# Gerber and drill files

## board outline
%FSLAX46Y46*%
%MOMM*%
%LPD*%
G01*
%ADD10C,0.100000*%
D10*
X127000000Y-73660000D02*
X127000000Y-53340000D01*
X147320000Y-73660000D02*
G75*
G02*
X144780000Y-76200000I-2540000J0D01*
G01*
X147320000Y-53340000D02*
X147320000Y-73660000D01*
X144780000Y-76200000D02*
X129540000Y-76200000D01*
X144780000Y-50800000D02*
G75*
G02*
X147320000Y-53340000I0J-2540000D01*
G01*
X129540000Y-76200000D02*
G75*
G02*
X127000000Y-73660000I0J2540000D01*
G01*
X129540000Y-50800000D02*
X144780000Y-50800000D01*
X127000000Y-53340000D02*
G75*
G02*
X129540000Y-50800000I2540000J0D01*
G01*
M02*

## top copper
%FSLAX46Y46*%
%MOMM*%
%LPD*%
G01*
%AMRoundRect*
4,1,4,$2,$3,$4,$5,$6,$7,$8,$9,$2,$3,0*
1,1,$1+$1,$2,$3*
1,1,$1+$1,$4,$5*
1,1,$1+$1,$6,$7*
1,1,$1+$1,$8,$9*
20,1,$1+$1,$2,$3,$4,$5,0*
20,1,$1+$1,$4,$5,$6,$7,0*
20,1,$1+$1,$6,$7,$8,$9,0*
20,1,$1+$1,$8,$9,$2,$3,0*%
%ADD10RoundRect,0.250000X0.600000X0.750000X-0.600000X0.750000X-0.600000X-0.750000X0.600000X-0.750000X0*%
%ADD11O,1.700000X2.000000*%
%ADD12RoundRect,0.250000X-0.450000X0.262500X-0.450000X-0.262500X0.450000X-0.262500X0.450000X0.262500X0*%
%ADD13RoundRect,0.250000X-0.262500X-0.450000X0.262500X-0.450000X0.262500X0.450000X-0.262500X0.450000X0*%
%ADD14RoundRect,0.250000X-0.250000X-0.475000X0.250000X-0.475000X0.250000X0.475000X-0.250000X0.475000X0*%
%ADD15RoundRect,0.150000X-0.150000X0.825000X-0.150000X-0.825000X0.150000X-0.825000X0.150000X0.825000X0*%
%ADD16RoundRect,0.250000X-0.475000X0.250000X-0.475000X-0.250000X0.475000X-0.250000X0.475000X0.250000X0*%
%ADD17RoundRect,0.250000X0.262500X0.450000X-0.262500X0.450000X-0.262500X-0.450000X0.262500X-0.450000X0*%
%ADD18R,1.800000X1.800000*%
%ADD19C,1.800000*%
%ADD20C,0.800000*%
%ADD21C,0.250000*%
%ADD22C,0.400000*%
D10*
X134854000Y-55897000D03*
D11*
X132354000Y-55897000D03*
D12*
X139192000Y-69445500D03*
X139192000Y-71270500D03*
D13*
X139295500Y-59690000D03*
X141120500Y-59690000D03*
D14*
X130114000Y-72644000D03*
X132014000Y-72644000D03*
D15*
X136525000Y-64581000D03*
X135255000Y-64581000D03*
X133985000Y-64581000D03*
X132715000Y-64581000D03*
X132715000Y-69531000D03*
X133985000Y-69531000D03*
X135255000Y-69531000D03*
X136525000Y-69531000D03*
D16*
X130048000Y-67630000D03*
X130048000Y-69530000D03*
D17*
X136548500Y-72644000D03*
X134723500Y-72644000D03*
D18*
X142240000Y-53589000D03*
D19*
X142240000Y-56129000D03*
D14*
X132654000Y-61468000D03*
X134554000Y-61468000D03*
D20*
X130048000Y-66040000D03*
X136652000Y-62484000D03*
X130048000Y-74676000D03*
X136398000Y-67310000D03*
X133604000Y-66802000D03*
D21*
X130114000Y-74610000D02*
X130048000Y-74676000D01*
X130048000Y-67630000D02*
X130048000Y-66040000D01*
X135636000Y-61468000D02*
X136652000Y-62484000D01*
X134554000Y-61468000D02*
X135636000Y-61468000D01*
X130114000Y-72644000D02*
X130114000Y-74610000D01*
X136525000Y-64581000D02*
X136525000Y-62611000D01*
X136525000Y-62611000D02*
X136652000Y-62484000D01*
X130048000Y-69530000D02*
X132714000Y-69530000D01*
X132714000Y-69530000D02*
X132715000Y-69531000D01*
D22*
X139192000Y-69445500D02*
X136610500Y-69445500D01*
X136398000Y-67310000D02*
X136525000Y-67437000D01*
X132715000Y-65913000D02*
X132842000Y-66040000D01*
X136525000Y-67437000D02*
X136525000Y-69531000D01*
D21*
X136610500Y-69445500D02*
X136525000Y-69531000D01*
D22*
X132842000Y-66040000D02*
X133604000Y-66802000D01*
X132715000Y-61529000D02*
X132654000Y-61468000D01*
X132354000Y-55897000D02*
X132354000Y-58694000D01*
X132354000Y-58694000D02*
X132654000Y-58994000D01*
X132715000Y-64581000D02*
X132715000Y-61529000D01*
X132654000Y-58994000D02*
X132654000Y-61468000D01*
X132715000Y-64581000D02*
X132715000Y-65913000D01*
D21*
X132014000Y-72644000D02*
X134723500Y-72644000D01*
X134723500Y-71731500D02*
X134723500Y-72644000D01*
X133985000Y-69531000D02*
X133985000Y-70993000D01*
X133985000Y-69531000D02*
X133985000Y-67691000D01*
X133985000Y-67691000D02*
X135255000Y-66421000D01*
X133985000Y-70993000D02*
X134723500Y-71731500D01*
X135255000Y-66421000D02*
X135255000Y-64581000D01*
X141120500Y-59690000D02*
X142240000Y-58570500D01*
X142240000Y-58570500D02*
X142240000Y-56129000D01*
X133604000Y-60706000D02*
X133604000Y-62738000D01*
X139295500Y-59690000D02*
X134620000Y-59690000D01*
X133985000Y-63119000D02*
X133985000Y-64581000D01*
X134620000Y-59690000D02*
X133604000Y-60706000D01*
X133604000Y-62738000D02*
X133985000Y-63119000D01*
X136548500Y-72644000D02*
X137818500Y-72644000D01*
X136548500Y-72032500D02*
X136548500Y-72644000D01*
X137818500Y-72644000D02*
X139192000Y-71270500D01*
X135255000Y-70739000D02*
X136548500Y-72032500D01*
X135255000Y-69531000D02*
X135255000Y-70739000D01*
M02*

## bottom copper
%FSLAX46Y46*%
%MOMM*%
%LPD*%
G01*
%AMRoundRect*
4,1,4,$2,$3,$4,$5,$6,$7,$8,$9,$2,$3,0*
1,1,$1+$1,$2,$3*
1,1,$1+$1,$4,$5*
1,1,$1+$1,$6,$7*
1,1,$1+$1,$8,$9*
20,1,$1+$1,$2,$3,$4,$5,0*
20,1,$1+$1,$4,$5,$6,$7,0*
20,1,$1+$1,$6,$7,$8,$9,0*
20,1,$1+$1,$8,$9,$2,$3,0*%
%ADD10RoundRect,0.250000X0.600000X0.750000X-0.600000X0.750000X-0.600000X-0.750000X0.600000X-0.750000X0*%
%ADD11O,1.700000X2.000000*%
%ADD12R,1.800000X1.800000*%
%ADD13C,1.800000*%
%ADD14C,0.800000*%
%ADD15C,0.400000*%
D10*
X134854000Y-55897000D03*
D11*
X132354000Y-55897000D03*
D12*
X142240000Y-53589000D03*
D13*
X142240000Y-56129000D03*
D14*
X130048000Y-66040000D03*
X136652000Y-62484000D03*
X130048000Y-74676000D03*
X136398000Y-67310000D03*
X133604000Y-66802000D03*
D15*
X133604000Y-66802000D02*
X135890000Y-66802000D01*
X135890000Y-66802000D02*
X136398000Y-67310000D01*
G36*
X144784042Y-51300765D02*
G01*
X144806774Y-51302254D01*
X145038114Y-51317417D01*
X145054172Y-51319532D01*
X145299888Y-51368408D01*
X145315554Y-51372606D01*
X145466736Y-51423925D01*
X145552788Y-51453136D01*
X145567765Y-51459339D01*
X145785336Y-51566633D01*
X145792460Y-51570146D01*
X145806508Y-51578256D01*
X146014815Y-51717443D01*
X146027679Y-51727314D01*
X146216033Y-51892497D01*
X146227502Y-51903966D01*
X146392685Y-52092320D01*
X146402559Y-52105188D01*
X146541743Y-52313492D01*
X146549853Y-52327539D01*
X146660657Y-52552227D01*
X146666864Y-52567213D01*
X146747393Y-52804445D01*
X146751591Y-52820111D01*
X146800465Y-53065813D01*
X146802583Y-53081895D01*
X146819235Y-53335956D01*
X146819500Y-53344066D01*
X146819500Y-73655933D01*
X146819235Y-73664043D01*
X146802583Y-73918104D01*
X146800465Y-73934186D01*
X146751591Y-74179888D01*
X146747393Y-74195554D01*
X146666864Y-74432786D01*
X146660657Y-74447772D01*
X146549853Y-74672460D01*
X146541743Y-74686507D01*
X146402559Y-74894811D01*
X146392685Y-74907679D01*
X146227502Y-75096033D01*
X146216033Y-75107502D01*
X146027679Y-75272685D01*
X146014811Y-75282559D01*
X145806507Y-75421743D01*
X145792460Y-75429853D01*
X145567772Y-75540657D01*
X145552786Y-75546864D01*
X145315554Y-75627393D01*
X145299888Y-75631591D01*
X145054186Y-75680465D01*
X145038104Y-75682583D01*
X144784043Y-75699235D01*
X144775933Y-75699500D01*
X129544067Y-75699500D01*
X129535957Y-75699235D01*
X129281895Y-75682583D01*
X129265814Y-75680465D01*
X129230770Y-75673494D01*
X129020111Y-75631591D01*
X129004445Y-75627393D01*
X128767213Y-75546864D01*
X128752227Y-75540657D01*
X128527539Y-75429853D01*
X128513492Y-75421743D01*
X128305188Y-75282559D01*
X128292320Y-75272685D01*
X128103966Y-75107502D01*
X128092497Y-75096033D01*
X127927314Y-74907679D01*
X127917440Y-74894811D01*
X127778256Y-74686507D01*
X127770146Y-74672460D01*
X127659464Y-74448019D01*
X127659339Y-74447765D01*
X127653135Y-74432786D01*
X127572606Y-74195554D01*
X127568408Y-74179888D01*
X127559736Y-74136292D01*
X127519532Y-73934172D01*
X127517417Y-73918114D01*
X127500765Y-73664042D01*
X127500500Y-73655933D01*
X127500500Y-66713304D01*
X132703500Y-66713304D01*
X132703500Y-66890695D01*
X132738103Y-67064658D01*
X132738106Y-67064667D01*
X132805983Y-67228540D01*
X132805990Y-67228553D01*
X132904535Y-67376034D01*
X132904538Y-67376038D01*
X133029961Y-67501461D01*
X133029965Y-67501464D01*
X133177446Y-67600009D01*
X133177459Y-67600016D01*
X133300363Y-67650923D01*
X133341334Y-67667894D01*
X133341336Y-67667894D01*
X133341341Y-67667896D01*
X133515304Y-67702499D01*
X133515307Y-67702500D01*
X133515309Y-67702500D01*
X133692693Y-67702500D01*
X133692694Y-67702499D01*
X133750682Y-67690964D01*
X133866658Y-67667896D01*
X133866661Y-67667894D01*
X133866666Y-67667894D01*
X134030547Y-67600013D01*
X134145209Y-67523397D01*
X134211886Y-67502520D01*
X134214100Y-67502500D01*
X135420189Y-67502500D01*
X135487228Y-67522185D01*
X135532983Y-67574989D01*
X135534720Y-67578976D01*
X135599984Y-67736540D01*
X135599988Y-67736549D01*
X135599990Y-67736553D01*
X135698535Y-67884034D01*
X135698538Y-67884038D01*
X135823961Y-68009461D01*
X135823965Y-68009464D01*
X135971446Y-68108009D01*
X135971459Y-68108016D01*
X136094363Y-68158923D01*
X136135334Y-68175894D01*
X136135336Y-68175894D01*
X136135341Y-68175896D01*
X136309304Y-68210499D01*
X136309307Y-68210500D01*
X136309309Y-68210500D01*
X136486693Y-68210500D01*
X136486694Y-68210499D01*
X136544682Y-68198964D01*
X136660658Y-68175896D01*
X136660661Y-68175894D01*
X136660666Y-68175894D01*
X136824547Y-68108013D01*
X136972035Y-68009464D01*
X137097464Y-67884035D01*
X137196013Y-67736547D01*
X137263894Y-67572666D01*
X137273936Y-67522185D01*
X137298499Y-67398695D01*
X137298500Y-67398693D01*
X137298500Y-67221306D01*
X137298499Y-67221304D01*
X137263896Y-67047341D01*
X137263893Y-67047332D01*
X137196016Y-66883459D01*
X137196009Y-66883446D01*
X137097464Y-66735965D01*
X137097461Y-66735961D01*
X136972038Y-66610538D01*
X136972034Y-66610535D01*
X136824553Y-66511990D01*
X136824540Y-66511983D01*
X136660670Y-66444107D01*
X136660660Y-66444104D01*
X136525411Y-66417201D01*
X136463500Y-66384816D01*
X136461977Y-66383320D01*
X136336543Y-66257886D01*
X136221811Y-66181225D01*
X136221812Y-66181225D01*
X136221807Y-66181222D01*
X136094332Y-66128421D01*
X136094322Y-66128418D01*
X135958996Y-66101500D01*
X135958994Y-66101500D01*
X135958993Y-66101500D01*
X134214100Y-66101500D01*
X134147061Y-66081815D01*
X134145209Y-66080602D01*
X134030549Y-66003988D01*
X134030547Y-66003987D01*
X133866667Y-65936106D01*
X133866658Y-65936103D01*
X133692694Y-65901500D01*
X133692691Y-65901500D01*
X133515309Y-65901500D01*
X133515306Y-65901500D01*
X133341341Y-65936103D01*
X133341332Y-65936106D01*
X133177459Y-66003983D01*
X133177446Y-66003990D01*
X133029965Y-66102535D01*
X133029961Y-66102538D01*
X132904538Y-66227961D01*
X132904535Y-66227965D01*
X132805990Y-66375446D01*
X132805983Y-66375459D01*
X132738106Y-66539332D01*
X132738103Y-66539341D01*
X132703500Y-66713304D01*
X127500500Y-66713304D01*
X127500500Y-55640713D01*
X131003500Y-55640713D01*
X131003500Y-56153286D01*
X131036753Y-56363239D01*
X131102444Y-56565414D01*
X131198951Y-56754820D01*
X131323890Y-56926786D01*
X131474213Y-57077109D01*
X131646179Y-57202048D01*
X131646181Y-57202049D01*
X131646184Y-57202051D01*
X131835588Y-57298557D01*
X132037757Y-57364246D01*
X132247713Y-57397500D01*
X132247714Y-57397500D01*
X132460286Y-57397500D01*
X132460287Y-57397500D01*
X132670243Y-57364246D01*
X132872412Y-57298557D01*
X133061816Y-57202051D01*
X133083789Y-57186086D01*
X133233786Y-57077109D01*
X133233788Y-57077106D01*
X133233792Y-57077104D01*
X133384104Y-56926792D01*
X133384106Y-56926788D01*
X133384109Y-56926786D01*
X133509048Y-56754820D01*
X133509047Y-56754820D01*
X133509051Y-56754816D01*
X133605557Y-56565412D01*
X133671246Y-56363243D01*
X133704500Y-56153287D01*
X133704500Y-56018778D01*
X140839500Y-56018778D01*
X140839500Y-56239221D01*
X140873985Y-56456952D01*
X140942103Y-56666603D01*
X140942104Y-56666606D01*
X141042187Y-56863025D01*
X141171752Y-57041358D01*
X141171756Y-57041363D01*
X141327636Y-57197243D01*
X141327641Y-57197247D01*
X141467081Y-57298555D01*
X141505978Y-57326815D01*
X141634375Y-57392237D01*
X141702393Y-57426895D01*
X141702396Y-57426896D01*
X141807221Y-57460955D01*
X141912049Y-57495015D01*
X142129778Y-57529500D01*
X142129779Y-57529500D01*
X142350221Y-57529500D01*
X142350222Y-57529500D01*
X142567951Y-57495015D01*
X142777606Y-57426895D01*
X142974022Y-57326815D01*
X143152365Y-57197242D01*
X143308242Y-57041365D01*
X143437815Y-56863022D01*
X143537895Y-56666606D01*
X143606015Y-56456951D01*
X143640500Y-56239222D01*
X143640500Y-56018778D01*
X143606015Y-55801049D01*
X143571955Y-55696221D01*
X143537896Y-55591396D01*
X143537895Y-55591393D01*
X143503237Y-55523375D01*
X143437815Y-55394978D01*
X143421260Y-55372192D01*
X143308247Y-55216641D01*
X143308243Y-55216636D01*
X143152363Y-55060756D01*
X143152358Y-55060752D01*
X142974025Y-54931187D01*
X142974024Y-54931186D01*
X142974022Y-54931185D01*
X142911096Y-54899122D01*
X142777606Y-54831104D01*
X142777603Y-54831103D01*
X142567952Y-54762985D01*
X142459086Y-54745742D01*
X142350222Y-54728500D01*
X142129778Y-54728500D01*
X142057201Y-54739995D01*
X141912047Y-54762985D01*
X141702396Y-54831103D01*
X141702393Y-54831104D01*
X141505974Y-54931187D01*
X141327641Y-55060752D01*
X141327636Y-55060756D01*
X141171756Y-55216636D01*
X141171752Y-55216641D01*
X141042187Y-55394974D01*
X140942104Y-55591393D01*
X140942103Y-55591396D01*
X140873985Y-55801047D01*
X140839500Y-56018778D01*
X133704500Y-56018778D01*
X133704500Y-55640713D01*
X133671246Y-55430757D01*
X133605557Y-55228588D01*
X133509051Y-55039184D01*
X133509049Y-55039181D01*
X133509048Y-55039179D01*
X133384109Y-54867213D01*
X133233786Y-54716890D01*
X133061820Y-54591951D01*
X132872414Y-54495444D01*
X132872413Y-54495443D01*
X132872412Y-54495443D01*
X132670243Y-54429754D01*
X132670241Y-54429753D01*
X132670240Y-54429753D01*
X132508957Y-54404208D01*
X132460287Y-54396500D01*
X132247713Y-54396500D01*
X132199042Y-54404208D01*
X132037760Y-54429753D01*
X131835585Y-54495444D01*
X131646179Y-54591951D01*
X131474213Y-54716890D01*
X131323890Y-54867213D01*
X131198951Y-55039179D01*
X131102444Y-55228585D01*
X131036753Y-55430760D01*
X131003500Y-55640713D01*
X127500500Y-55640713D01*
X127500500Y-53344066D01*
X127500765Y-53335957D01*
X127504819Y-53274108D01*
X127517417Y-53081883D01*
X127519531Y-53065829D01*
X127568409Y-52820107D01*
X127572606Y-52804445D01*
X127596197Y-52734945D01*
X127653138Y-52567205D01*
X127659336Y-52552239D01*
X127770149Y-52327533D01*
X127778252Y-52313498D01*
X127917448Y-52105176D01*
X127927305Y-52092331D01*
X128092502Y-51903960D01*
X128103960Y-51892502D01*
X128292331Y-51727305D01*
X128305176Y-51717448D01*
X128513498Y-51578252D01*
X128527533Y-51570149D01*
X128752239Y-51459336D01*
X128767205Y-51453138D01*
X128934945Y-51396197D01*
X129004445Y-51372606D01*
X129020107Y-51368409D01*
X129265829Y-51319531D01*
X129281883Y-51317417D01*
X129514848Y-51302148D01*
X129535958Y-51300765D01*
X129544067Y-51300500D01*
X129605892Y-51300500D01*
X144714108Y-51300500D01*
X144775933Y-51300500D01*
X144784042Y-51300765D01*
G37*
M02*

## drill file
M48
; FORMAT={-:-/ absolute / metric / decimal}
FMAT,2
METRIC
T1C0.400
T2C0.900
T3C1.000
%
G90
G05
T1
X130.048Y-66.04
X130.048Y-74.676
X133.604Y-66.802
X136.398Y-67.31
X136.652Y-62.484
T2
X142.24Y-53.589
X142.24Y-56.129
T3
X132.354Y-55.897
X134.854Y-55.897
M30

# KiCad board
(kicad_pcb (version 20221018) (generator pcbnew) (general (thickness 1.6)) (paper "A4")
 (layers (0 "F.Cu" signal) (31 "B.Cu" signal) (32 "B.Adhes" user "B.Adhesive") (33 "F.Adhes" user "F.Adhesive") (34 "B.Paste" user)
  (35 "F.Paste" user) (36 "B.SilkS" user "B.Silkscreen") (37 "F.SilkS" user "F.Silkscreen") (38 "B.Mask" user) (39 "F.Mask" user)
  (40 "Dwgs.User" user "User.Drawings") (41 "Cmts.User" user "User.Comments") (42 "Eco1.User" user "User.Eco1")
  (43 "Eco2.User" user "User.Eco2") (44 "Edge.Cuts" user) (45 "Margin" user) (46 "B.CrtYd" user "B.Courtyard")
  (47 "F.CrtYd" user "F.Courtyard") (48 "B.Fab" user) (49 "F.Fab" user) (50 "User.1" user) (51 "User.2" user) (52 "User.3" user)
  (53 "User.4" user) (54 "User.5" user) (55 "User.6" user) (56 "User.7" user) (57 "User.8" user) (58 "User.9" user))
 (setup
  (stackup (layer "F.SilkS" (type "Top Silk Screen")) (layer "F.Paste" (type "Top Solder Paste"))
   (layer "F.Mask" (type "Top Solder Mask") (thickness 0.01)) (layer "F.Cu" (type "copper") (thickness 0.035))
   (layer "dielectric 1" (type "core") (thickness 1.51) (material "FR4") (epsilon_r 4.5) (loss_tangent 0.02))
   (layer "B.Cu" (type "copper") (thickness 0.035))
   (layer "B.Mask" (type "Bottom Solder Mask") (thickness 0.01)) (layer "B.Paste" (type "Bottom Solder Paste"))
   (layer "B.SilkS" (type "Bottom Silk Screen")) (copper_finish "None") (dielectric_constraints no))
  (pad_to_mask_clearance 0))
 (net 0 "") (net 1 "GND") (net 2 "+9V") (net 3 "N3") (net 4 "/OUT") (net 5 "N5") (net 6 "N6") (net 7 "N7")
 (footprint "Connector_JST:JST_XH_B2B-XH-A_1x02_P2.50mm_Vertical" (layer "F.Cu") (at 134.854 55.897 180)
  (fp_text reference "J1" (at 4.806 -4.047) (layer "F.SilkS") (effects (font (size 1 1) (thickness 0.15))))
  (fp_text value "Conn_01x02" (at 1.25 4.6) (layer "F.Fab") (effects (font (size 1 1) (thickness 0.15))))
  (pad "1" thru_hole roundrect (at 0 0 180) (size 1.7 2) (drill 1) (layers "*.Cu" "*.Mask") (roundrect_rratio 0.1470588235) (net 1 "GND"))
  (pad "2" thru_hole oval (at 2.5 0 180) (size 1.7 2) (drill 1) (layers "*.Cu" "*.Mask") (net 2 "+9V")))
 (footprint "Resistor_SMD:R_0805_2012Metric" (layer "F.Cu") (at 139.192 70.358 -90)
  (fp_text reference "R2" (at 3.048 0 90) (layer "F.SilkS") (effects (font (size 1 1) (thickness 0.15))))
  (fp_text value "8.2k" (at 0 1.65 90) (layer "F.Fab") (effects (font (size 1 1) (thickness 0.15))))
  (pad "1" smd roundrect (at -0.9125 0 270) (size 1.025 1.4) (layers "F.Cu" "F.Paste" "F.Mask") (roundrect_rratio 0.243902439) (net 2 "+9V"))
  (pad "2" smd roundrect (at 0.9125 0 270) (size 1.025 1.4) (layers "F.Cu" "F.Paste" "F.Mask") (roundrect_rratio 0.243902439) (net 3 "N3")))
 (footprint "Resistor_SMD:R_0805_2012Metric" (layer "F.Cu") (at 140.208 59.69)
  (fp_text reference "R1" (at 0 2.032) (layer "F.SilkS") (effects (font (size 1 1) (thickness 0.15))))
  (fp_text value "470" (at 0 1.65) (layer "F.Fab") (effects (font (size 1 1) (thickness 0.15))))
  (pad "1" smd roundrect (at -0.9125 0) (size 1.025 1.4) (layers "F.Cu" "F.Paste" "F.Mask") (roundrect_rratio 0.243902439) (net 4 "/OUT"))
  (pad "2" smd roundrect (at 0.9125 0) (size 1.025 1.4) (layers "F.Cu" "F.Paste" "F.Mask") (roundrect_rratio 0.243902439) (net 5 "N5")))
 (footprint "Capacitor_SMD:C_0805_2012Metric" (layer "F.Cu") (at 131.064 72.644)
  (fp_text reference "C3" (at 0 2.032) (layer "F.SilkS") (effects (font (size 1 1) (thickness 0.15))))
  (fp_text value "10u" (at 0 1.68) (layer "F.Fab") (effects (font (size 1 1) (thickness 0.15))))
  (pad "1" smd roundrect (at -0.95 0) (size 1 1.45) (layers "F.Cu" "F.Paste" "F.Mask") (roundrect_rratio 0.25) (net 1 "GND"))
  (pad "2" smd roundrect (at 0.95 0) (size 1 1.45) (layers "F.Cu" "F.Paste" "F.Mask") (roundrect_rratio 0.25) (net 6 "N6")))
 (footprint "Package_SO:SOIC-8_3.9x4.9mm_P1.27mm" (layer "F.Cu") (at 134.62 67.056 -90)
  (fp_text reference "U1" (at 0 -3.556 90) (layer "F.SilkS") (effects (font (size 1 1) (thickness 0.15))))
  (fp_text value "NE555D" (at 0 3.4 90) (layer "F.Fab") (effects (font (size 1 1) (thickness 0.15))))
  (pad "1" smd roundrect (at -2.475 -1.905 270) (size 1.95 0.6) (layers "F.Cu" "F.Paste" "F.Mask") (roundrect_rratio 0.25) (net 1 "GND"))
  (pad "2" smd roundrect (at -2.475 -0.635 270) (size 1.95 0.6) (layers "F.Cu" "F.Paste" "F.Mask") (roundrect_rratio 0.25) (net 6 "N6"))
  (pad "3" smd roundrect (at -2.475 0.635 270) (size 1.95 0.6) (layers "F.Cu" "F.Paste" "F.Mask") (roundrect_rratio 0.25) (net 4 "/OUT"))
  (pad "4" smd roundrect (at -2.475 1.905 270) (size 1.95 0.6) (layers "F.Cu" "F.Paste" "F.Mask") (roundrect_rratio 0.25) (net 2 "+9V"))
  (pad "5" smd roundrect (at 2.475 1.905 270) (size 1.95 0.6) (layers "F.Cu" "F.Paste" "F.Mask") (roundrect_rratio 0.25) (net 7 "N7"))
  (pad "6" smd roundrect (at 2.475 0.635 270) (size 1.95 0.6) (layers "F.Cu" "F.Paste" "F.Mask") (roundrect_rratio 0.25) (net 6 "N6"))
  (pad "7" smd roundrect (at 2.475 -0.635 270) (size 1.95 0.6) (layers "F.Cu" "F.Paste" "F.Mask") (roundrect_rratio 0.25) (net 3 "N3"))
  (pad "8" smd roundrect (at 2.475 -1.905 270) (size 1.95 0.6) (layers "F.Cu" "F.Paste" "F.Mask") (roundrect_rratio 0.25) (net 2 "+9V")))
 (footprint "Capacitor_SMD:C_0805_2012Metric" (layer "F.Cu") (at 130.048 68.58 -90)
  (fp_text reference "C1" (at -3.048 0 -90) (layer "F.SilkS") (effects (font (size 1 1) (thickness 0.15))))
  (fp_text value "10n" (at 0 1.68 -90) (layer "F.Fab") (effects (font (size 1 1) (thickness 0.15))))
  (pad "1" smd roundrect (at -0.95 0 270) (size 1 1.45) (layers "F.Cu" "F.Paste" "F.Mask") (roundrect_rratio 0.25) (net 1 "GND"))
  (pad "2" smd roundrect (at 0.95 0 270) (size 1 1.45) (layers "F.Cu" "F.Paste" "F.Mask") (roundrect_rratio 0.25) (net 7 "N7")))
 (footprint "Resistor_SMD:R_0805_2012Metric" (layer "F.Cu") (at 135.636 72.644 180)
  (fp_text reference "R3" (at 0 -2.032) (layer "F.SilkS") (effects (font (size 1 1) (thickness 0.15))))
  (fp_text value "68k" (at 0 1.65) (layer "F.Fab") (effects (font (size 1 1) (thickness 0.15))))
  (pad "1" smd roundrect (at -0.9125 0 180) (size 1.025 1.4) (layers "F.Cu" "F.Paste" "F.Mask") (roundrect_rratio 0.243902439) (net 3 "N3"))
  (pad "2" smd roundrect (at 0.9125 0 180) (size 1.025 1.4) (layers "F.Cu" "F.Paste" "F.Mask") (roundrect_rratio 0.243902439) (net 6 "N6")))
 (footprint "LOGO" (layer "F.Cu") (at 142.748 67.31 90)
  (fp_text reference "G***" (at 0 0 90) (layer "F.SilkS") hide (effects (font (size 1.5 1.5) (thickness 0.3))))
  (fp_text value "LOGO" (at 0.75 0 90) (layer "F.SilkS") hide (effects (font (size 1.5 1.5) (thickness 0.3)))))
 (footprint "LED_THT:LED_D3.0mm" (layer "F.Cu") (at 142.24 53.589 -90)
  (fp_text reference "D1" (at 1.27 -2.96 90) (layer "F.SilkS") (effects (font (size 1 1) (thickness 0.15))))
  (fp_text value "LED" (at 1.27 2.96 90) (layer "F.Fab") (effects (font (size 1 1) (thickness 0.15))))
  (pad "1" thru_hole rect (at 0 0 270) (size 1.8 1.8) (drill 0.9) (layers "*.Cu" "*.Mask") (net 1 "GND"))
  (pad "2" thru_hole circle (at 2.54 0 270) (size 1.8 1.8) (drill 0.9) (layers "*.Cu" "*.Mask") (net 5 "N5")))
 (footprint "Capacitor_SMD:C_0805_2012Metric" (layer "F.Cu") (at 133.604 61.468)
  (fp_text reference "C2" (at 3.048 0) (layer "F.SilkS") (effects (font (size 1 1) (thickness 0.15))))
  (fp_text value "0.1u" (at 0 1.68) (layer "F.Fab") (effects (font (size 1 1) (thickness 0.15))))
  (pad "1" smd roundrect (at -0.95 0) (size 1 1.45) (layers "F.Cu" "F.Paste" "F.Mask") (roundrect_rratio 0.25) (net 2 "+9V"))
  (pad "2" smd roundrect (at 0.95 0) (size 1 1.45) (layers "F.Cu" "F.Paste" "F.Mask") (roundrect_rratio 0.25) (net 1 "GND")))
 (gr_line (start 127 73.66) (end 127 53.34) (stroke (width 0.1) (type default)) (layer "Edge.Cuts"))
 (gr_arc (start 147.32 73.66) (mid 146.576051 75.456051) (end 144.78 76.2) (stroke (width 0.1) (type default)) (layer "Edge.Cuts"))
 (gr_line (start 147.32 53.34) (end 147.32 73.66) (stroke (width 0.1) (type default)) (layer "Edge.Cuts"))
 (gr_line (start 144.78 76.2) (end 129.54 76.2) (stroke (width 0.1) (type default)) (layer "Edge.Cuts"))
 (gr_arc (start 144.78 50.8) (mid 146.576051 51.543949) (end 147.32 53.34) (stroke (width 0.1) (type default)) (layer "Edge.Cuts"))
 (gr_arc (start 129.54 76.2) (mid 127.743949 75.456051) (end 127 73.66) (stroke (width 0.1) (type default)) (layer "Edge.Cuts"))
 (gr_line (start 129.54 50.8) (end 144.78 50.8) (stroke (width 0.1) (type default)) (layer "Edge.Cuts"))
 (gr_arc (start 127 53.34) (mid 127.743949 51.543949) (end 129.54 50.8) (stroke (width 0.1) (type default)) (layer "Edge.Cuts"))
 (segment (start 130.114 74.61) (end 130.048 74.676) (width 0.25) (layer "F.Cu") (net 1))
 (segment (start 130.048 67.63) (end 130.048 66.04) (width 0.25) (layer "F.Cu") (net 1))
 (segment (start 135.636 61.468) (end 136.652 62.484) (width 0.25) (layer "F.Cu") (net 1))
 (segment (start 134.554 61.468) (end 135.636 61.468) (width 0.25) (layer "F.Cu") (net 1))
 (segment (start 130.114 72.644) (end 130.114 74.61) (width 0.25) (layer "F.Cu") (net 1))
 (segment (start 136.525 64.581) (end 136.525 62.611) (width 0.25) (layer "F.Cu") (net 1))
 (segment (start 136.525 62.611) (end 136.652 62.484) (width 0.25) (layer "F.Cu") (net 1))
 (via (at 130.048 66.04) (size 0.8) (drill 0.4) (layers "F.Cu" "B.Cu") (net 1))
 (via (at 136.652 62.484) (size 0.8) (drill 0.4) (layers "F.Cu" "B.Cu") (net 1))
 (via (at 130.048 74.676) (size 0.8) (drill 0.4) (layers "F.Cu" "B.Cu") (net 1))
 (segment (start 130.048 69.53) (end 132.714 69.53) (width 0.25) (layer "F.Cu") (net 7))
 (segment (start 132.714 69.53) (end 132.715 69.531) (width 0.25) (layer "F.Cu") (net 7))
 (segment (start 139.192 69.4455) (end 136.6105 69.4455) (width 0.4) (layer "F.Cu") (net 2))
 (segment (start 136.398 67.31) (end 136.525 67.437) (width 0.4) (layer "F.Cu") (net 2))
 (segment (start 132.715 65.913) (end 132.842 66.04) (width 0.4) (layer "F.Cu") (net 2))
 (segment (start 136.525 67.437) (end 136.525 69.531) (width 0.4) (layer "F.Cu") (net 2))
 (segment (start 136.6105 69.4455) (end 136.525 69.531) (width 0.25) (layer "F.Cu") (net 2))
 (segment (start 132.842 66.04) (end 133.604 66.802) (width 0.4) (layer "F.Cu") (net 2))
 (segment (start 132.715 61.529) (end 132.654 61.468) (width 0.4) (layer "F.Cu") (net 2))
 (segment (start 132.354 55.897) (end 132.354 58.694) (width 0.4) (layer "F.Cu") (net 2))
 (segment (start 132.354 58.694) (end 132.654 58.994) (width 0.4) (layer "F.Cu") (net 2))
 (segment (start 132.715 64.581) (end 132.715 61.529) (width 0.4) (layer "F.Cu") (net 2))
 (segment (start 132.654 58.994) (end 132.654 61.468) (width 0.4) (layer "F.Cu") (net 2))
 (segment (start 132.715 64.581) (end 132.715 65.913) (width 0.4) (layer "F.Cu") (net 2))
 (via (at 136.398 67.31) (size 0.8) (drill 0.4) (layers "F.Cu" "B.Cu") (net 2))
 (via (at 133.604 66.802) (size 0.8) (drill 0.4) (layers "F.Cu" "B.Cu") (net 2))
 (segment (start 133.604 66.802) (end 135.89 66.802) (width 0.4) (layer "B.Cu") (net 2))
 (segment (start 135.89 66.802) (end 136.398 67.31) (width 0.4) (layer "B.Cu") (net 2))
 (segment (start 132.014 72.644) (end 134.7235 72.644) (width 0.25) (layer "F.Cu") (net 6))
 (segment (start 134.7235 71.7315) (end 134.7235 72.644) (width 0.25) (layer "F.Cu") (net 6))
 (segment (start 133.985 69.531) (end 133.985 70.993) (width 0.25) (layer "F.Cu") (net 6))
 (segment (start 133.985 69.531) (end 133.985 67.691) (width 0.25) (layer "F.Cu") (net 6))
 (segment (start 133.985 67.691) (end 135.255 66.421) (width 0.25) (layer "F.Cu") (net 6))
 (segment (start 133.985 70.993) (end 134.7235 71.7315) (width 0.25) (layer "F.Cu") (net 6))
 (segment (start 135.255 66.421) (end 135.255 64.581) (width 0.25) (layer "F.Cu") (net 6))
 (segment (start 141.1205 59.69) (end 142.24 58.5705) (width 0.25) (layer "F.Cu") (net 5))
 (segment (start 142.24 58.5705) (end 142.24 56.129) (width 0.25) (layer "F.Cu") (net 5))
 (segment (start 133.604 60.706) (end 133.604 62.738) (width 0.25) (layer "F.Cu") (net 4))
 (segment (start 139.2955 59.69) (end 134.62 59.69) (width 0.25) (layer "F.Cu") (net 4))
 (segment (start 133.985 63.119) (end 133.985 64.581) (width 0.25) (layer "F.Cu") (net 4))
 (segment (start 134.62 59.69) (end 133.604 60.706) (width 0.25) (layer "F.Cu") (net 4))
 (segment (start 133.604 62.738) (end 133.985 63.119) (width 0.25) (layer "F.Cu") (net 4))
 (segment (start 136.5485 72.644) (end 137.8185 72.644) (width 0.25) (layer "F.Cu") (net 3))
 (segment (start 136.5485 72.0325) (end 136.5485 72.644) (width 0.25) (layer "F.Cu") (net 3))
 (segment (start 137.8185 72.644) (end 139.192 71.2705) (width 0.25) (layer "F.Cu") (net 3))
 (segment (start 135.255 70.739) (end 136.5485 72.0325) (width 0.25) (layer "F.Cu") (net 3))
 (segment (start 135.255 69.531) (end 135.255 70.739) (width 0.25) (layer "F.Cu") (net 3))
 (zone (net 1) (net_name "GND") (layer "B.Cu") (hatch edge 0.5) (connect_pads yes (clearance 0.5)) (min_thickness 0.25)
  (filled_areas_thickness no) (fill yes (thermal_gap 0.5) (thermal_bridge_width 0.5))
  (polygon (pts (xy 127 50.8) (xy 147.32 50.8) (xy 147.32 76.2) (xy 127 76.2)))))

